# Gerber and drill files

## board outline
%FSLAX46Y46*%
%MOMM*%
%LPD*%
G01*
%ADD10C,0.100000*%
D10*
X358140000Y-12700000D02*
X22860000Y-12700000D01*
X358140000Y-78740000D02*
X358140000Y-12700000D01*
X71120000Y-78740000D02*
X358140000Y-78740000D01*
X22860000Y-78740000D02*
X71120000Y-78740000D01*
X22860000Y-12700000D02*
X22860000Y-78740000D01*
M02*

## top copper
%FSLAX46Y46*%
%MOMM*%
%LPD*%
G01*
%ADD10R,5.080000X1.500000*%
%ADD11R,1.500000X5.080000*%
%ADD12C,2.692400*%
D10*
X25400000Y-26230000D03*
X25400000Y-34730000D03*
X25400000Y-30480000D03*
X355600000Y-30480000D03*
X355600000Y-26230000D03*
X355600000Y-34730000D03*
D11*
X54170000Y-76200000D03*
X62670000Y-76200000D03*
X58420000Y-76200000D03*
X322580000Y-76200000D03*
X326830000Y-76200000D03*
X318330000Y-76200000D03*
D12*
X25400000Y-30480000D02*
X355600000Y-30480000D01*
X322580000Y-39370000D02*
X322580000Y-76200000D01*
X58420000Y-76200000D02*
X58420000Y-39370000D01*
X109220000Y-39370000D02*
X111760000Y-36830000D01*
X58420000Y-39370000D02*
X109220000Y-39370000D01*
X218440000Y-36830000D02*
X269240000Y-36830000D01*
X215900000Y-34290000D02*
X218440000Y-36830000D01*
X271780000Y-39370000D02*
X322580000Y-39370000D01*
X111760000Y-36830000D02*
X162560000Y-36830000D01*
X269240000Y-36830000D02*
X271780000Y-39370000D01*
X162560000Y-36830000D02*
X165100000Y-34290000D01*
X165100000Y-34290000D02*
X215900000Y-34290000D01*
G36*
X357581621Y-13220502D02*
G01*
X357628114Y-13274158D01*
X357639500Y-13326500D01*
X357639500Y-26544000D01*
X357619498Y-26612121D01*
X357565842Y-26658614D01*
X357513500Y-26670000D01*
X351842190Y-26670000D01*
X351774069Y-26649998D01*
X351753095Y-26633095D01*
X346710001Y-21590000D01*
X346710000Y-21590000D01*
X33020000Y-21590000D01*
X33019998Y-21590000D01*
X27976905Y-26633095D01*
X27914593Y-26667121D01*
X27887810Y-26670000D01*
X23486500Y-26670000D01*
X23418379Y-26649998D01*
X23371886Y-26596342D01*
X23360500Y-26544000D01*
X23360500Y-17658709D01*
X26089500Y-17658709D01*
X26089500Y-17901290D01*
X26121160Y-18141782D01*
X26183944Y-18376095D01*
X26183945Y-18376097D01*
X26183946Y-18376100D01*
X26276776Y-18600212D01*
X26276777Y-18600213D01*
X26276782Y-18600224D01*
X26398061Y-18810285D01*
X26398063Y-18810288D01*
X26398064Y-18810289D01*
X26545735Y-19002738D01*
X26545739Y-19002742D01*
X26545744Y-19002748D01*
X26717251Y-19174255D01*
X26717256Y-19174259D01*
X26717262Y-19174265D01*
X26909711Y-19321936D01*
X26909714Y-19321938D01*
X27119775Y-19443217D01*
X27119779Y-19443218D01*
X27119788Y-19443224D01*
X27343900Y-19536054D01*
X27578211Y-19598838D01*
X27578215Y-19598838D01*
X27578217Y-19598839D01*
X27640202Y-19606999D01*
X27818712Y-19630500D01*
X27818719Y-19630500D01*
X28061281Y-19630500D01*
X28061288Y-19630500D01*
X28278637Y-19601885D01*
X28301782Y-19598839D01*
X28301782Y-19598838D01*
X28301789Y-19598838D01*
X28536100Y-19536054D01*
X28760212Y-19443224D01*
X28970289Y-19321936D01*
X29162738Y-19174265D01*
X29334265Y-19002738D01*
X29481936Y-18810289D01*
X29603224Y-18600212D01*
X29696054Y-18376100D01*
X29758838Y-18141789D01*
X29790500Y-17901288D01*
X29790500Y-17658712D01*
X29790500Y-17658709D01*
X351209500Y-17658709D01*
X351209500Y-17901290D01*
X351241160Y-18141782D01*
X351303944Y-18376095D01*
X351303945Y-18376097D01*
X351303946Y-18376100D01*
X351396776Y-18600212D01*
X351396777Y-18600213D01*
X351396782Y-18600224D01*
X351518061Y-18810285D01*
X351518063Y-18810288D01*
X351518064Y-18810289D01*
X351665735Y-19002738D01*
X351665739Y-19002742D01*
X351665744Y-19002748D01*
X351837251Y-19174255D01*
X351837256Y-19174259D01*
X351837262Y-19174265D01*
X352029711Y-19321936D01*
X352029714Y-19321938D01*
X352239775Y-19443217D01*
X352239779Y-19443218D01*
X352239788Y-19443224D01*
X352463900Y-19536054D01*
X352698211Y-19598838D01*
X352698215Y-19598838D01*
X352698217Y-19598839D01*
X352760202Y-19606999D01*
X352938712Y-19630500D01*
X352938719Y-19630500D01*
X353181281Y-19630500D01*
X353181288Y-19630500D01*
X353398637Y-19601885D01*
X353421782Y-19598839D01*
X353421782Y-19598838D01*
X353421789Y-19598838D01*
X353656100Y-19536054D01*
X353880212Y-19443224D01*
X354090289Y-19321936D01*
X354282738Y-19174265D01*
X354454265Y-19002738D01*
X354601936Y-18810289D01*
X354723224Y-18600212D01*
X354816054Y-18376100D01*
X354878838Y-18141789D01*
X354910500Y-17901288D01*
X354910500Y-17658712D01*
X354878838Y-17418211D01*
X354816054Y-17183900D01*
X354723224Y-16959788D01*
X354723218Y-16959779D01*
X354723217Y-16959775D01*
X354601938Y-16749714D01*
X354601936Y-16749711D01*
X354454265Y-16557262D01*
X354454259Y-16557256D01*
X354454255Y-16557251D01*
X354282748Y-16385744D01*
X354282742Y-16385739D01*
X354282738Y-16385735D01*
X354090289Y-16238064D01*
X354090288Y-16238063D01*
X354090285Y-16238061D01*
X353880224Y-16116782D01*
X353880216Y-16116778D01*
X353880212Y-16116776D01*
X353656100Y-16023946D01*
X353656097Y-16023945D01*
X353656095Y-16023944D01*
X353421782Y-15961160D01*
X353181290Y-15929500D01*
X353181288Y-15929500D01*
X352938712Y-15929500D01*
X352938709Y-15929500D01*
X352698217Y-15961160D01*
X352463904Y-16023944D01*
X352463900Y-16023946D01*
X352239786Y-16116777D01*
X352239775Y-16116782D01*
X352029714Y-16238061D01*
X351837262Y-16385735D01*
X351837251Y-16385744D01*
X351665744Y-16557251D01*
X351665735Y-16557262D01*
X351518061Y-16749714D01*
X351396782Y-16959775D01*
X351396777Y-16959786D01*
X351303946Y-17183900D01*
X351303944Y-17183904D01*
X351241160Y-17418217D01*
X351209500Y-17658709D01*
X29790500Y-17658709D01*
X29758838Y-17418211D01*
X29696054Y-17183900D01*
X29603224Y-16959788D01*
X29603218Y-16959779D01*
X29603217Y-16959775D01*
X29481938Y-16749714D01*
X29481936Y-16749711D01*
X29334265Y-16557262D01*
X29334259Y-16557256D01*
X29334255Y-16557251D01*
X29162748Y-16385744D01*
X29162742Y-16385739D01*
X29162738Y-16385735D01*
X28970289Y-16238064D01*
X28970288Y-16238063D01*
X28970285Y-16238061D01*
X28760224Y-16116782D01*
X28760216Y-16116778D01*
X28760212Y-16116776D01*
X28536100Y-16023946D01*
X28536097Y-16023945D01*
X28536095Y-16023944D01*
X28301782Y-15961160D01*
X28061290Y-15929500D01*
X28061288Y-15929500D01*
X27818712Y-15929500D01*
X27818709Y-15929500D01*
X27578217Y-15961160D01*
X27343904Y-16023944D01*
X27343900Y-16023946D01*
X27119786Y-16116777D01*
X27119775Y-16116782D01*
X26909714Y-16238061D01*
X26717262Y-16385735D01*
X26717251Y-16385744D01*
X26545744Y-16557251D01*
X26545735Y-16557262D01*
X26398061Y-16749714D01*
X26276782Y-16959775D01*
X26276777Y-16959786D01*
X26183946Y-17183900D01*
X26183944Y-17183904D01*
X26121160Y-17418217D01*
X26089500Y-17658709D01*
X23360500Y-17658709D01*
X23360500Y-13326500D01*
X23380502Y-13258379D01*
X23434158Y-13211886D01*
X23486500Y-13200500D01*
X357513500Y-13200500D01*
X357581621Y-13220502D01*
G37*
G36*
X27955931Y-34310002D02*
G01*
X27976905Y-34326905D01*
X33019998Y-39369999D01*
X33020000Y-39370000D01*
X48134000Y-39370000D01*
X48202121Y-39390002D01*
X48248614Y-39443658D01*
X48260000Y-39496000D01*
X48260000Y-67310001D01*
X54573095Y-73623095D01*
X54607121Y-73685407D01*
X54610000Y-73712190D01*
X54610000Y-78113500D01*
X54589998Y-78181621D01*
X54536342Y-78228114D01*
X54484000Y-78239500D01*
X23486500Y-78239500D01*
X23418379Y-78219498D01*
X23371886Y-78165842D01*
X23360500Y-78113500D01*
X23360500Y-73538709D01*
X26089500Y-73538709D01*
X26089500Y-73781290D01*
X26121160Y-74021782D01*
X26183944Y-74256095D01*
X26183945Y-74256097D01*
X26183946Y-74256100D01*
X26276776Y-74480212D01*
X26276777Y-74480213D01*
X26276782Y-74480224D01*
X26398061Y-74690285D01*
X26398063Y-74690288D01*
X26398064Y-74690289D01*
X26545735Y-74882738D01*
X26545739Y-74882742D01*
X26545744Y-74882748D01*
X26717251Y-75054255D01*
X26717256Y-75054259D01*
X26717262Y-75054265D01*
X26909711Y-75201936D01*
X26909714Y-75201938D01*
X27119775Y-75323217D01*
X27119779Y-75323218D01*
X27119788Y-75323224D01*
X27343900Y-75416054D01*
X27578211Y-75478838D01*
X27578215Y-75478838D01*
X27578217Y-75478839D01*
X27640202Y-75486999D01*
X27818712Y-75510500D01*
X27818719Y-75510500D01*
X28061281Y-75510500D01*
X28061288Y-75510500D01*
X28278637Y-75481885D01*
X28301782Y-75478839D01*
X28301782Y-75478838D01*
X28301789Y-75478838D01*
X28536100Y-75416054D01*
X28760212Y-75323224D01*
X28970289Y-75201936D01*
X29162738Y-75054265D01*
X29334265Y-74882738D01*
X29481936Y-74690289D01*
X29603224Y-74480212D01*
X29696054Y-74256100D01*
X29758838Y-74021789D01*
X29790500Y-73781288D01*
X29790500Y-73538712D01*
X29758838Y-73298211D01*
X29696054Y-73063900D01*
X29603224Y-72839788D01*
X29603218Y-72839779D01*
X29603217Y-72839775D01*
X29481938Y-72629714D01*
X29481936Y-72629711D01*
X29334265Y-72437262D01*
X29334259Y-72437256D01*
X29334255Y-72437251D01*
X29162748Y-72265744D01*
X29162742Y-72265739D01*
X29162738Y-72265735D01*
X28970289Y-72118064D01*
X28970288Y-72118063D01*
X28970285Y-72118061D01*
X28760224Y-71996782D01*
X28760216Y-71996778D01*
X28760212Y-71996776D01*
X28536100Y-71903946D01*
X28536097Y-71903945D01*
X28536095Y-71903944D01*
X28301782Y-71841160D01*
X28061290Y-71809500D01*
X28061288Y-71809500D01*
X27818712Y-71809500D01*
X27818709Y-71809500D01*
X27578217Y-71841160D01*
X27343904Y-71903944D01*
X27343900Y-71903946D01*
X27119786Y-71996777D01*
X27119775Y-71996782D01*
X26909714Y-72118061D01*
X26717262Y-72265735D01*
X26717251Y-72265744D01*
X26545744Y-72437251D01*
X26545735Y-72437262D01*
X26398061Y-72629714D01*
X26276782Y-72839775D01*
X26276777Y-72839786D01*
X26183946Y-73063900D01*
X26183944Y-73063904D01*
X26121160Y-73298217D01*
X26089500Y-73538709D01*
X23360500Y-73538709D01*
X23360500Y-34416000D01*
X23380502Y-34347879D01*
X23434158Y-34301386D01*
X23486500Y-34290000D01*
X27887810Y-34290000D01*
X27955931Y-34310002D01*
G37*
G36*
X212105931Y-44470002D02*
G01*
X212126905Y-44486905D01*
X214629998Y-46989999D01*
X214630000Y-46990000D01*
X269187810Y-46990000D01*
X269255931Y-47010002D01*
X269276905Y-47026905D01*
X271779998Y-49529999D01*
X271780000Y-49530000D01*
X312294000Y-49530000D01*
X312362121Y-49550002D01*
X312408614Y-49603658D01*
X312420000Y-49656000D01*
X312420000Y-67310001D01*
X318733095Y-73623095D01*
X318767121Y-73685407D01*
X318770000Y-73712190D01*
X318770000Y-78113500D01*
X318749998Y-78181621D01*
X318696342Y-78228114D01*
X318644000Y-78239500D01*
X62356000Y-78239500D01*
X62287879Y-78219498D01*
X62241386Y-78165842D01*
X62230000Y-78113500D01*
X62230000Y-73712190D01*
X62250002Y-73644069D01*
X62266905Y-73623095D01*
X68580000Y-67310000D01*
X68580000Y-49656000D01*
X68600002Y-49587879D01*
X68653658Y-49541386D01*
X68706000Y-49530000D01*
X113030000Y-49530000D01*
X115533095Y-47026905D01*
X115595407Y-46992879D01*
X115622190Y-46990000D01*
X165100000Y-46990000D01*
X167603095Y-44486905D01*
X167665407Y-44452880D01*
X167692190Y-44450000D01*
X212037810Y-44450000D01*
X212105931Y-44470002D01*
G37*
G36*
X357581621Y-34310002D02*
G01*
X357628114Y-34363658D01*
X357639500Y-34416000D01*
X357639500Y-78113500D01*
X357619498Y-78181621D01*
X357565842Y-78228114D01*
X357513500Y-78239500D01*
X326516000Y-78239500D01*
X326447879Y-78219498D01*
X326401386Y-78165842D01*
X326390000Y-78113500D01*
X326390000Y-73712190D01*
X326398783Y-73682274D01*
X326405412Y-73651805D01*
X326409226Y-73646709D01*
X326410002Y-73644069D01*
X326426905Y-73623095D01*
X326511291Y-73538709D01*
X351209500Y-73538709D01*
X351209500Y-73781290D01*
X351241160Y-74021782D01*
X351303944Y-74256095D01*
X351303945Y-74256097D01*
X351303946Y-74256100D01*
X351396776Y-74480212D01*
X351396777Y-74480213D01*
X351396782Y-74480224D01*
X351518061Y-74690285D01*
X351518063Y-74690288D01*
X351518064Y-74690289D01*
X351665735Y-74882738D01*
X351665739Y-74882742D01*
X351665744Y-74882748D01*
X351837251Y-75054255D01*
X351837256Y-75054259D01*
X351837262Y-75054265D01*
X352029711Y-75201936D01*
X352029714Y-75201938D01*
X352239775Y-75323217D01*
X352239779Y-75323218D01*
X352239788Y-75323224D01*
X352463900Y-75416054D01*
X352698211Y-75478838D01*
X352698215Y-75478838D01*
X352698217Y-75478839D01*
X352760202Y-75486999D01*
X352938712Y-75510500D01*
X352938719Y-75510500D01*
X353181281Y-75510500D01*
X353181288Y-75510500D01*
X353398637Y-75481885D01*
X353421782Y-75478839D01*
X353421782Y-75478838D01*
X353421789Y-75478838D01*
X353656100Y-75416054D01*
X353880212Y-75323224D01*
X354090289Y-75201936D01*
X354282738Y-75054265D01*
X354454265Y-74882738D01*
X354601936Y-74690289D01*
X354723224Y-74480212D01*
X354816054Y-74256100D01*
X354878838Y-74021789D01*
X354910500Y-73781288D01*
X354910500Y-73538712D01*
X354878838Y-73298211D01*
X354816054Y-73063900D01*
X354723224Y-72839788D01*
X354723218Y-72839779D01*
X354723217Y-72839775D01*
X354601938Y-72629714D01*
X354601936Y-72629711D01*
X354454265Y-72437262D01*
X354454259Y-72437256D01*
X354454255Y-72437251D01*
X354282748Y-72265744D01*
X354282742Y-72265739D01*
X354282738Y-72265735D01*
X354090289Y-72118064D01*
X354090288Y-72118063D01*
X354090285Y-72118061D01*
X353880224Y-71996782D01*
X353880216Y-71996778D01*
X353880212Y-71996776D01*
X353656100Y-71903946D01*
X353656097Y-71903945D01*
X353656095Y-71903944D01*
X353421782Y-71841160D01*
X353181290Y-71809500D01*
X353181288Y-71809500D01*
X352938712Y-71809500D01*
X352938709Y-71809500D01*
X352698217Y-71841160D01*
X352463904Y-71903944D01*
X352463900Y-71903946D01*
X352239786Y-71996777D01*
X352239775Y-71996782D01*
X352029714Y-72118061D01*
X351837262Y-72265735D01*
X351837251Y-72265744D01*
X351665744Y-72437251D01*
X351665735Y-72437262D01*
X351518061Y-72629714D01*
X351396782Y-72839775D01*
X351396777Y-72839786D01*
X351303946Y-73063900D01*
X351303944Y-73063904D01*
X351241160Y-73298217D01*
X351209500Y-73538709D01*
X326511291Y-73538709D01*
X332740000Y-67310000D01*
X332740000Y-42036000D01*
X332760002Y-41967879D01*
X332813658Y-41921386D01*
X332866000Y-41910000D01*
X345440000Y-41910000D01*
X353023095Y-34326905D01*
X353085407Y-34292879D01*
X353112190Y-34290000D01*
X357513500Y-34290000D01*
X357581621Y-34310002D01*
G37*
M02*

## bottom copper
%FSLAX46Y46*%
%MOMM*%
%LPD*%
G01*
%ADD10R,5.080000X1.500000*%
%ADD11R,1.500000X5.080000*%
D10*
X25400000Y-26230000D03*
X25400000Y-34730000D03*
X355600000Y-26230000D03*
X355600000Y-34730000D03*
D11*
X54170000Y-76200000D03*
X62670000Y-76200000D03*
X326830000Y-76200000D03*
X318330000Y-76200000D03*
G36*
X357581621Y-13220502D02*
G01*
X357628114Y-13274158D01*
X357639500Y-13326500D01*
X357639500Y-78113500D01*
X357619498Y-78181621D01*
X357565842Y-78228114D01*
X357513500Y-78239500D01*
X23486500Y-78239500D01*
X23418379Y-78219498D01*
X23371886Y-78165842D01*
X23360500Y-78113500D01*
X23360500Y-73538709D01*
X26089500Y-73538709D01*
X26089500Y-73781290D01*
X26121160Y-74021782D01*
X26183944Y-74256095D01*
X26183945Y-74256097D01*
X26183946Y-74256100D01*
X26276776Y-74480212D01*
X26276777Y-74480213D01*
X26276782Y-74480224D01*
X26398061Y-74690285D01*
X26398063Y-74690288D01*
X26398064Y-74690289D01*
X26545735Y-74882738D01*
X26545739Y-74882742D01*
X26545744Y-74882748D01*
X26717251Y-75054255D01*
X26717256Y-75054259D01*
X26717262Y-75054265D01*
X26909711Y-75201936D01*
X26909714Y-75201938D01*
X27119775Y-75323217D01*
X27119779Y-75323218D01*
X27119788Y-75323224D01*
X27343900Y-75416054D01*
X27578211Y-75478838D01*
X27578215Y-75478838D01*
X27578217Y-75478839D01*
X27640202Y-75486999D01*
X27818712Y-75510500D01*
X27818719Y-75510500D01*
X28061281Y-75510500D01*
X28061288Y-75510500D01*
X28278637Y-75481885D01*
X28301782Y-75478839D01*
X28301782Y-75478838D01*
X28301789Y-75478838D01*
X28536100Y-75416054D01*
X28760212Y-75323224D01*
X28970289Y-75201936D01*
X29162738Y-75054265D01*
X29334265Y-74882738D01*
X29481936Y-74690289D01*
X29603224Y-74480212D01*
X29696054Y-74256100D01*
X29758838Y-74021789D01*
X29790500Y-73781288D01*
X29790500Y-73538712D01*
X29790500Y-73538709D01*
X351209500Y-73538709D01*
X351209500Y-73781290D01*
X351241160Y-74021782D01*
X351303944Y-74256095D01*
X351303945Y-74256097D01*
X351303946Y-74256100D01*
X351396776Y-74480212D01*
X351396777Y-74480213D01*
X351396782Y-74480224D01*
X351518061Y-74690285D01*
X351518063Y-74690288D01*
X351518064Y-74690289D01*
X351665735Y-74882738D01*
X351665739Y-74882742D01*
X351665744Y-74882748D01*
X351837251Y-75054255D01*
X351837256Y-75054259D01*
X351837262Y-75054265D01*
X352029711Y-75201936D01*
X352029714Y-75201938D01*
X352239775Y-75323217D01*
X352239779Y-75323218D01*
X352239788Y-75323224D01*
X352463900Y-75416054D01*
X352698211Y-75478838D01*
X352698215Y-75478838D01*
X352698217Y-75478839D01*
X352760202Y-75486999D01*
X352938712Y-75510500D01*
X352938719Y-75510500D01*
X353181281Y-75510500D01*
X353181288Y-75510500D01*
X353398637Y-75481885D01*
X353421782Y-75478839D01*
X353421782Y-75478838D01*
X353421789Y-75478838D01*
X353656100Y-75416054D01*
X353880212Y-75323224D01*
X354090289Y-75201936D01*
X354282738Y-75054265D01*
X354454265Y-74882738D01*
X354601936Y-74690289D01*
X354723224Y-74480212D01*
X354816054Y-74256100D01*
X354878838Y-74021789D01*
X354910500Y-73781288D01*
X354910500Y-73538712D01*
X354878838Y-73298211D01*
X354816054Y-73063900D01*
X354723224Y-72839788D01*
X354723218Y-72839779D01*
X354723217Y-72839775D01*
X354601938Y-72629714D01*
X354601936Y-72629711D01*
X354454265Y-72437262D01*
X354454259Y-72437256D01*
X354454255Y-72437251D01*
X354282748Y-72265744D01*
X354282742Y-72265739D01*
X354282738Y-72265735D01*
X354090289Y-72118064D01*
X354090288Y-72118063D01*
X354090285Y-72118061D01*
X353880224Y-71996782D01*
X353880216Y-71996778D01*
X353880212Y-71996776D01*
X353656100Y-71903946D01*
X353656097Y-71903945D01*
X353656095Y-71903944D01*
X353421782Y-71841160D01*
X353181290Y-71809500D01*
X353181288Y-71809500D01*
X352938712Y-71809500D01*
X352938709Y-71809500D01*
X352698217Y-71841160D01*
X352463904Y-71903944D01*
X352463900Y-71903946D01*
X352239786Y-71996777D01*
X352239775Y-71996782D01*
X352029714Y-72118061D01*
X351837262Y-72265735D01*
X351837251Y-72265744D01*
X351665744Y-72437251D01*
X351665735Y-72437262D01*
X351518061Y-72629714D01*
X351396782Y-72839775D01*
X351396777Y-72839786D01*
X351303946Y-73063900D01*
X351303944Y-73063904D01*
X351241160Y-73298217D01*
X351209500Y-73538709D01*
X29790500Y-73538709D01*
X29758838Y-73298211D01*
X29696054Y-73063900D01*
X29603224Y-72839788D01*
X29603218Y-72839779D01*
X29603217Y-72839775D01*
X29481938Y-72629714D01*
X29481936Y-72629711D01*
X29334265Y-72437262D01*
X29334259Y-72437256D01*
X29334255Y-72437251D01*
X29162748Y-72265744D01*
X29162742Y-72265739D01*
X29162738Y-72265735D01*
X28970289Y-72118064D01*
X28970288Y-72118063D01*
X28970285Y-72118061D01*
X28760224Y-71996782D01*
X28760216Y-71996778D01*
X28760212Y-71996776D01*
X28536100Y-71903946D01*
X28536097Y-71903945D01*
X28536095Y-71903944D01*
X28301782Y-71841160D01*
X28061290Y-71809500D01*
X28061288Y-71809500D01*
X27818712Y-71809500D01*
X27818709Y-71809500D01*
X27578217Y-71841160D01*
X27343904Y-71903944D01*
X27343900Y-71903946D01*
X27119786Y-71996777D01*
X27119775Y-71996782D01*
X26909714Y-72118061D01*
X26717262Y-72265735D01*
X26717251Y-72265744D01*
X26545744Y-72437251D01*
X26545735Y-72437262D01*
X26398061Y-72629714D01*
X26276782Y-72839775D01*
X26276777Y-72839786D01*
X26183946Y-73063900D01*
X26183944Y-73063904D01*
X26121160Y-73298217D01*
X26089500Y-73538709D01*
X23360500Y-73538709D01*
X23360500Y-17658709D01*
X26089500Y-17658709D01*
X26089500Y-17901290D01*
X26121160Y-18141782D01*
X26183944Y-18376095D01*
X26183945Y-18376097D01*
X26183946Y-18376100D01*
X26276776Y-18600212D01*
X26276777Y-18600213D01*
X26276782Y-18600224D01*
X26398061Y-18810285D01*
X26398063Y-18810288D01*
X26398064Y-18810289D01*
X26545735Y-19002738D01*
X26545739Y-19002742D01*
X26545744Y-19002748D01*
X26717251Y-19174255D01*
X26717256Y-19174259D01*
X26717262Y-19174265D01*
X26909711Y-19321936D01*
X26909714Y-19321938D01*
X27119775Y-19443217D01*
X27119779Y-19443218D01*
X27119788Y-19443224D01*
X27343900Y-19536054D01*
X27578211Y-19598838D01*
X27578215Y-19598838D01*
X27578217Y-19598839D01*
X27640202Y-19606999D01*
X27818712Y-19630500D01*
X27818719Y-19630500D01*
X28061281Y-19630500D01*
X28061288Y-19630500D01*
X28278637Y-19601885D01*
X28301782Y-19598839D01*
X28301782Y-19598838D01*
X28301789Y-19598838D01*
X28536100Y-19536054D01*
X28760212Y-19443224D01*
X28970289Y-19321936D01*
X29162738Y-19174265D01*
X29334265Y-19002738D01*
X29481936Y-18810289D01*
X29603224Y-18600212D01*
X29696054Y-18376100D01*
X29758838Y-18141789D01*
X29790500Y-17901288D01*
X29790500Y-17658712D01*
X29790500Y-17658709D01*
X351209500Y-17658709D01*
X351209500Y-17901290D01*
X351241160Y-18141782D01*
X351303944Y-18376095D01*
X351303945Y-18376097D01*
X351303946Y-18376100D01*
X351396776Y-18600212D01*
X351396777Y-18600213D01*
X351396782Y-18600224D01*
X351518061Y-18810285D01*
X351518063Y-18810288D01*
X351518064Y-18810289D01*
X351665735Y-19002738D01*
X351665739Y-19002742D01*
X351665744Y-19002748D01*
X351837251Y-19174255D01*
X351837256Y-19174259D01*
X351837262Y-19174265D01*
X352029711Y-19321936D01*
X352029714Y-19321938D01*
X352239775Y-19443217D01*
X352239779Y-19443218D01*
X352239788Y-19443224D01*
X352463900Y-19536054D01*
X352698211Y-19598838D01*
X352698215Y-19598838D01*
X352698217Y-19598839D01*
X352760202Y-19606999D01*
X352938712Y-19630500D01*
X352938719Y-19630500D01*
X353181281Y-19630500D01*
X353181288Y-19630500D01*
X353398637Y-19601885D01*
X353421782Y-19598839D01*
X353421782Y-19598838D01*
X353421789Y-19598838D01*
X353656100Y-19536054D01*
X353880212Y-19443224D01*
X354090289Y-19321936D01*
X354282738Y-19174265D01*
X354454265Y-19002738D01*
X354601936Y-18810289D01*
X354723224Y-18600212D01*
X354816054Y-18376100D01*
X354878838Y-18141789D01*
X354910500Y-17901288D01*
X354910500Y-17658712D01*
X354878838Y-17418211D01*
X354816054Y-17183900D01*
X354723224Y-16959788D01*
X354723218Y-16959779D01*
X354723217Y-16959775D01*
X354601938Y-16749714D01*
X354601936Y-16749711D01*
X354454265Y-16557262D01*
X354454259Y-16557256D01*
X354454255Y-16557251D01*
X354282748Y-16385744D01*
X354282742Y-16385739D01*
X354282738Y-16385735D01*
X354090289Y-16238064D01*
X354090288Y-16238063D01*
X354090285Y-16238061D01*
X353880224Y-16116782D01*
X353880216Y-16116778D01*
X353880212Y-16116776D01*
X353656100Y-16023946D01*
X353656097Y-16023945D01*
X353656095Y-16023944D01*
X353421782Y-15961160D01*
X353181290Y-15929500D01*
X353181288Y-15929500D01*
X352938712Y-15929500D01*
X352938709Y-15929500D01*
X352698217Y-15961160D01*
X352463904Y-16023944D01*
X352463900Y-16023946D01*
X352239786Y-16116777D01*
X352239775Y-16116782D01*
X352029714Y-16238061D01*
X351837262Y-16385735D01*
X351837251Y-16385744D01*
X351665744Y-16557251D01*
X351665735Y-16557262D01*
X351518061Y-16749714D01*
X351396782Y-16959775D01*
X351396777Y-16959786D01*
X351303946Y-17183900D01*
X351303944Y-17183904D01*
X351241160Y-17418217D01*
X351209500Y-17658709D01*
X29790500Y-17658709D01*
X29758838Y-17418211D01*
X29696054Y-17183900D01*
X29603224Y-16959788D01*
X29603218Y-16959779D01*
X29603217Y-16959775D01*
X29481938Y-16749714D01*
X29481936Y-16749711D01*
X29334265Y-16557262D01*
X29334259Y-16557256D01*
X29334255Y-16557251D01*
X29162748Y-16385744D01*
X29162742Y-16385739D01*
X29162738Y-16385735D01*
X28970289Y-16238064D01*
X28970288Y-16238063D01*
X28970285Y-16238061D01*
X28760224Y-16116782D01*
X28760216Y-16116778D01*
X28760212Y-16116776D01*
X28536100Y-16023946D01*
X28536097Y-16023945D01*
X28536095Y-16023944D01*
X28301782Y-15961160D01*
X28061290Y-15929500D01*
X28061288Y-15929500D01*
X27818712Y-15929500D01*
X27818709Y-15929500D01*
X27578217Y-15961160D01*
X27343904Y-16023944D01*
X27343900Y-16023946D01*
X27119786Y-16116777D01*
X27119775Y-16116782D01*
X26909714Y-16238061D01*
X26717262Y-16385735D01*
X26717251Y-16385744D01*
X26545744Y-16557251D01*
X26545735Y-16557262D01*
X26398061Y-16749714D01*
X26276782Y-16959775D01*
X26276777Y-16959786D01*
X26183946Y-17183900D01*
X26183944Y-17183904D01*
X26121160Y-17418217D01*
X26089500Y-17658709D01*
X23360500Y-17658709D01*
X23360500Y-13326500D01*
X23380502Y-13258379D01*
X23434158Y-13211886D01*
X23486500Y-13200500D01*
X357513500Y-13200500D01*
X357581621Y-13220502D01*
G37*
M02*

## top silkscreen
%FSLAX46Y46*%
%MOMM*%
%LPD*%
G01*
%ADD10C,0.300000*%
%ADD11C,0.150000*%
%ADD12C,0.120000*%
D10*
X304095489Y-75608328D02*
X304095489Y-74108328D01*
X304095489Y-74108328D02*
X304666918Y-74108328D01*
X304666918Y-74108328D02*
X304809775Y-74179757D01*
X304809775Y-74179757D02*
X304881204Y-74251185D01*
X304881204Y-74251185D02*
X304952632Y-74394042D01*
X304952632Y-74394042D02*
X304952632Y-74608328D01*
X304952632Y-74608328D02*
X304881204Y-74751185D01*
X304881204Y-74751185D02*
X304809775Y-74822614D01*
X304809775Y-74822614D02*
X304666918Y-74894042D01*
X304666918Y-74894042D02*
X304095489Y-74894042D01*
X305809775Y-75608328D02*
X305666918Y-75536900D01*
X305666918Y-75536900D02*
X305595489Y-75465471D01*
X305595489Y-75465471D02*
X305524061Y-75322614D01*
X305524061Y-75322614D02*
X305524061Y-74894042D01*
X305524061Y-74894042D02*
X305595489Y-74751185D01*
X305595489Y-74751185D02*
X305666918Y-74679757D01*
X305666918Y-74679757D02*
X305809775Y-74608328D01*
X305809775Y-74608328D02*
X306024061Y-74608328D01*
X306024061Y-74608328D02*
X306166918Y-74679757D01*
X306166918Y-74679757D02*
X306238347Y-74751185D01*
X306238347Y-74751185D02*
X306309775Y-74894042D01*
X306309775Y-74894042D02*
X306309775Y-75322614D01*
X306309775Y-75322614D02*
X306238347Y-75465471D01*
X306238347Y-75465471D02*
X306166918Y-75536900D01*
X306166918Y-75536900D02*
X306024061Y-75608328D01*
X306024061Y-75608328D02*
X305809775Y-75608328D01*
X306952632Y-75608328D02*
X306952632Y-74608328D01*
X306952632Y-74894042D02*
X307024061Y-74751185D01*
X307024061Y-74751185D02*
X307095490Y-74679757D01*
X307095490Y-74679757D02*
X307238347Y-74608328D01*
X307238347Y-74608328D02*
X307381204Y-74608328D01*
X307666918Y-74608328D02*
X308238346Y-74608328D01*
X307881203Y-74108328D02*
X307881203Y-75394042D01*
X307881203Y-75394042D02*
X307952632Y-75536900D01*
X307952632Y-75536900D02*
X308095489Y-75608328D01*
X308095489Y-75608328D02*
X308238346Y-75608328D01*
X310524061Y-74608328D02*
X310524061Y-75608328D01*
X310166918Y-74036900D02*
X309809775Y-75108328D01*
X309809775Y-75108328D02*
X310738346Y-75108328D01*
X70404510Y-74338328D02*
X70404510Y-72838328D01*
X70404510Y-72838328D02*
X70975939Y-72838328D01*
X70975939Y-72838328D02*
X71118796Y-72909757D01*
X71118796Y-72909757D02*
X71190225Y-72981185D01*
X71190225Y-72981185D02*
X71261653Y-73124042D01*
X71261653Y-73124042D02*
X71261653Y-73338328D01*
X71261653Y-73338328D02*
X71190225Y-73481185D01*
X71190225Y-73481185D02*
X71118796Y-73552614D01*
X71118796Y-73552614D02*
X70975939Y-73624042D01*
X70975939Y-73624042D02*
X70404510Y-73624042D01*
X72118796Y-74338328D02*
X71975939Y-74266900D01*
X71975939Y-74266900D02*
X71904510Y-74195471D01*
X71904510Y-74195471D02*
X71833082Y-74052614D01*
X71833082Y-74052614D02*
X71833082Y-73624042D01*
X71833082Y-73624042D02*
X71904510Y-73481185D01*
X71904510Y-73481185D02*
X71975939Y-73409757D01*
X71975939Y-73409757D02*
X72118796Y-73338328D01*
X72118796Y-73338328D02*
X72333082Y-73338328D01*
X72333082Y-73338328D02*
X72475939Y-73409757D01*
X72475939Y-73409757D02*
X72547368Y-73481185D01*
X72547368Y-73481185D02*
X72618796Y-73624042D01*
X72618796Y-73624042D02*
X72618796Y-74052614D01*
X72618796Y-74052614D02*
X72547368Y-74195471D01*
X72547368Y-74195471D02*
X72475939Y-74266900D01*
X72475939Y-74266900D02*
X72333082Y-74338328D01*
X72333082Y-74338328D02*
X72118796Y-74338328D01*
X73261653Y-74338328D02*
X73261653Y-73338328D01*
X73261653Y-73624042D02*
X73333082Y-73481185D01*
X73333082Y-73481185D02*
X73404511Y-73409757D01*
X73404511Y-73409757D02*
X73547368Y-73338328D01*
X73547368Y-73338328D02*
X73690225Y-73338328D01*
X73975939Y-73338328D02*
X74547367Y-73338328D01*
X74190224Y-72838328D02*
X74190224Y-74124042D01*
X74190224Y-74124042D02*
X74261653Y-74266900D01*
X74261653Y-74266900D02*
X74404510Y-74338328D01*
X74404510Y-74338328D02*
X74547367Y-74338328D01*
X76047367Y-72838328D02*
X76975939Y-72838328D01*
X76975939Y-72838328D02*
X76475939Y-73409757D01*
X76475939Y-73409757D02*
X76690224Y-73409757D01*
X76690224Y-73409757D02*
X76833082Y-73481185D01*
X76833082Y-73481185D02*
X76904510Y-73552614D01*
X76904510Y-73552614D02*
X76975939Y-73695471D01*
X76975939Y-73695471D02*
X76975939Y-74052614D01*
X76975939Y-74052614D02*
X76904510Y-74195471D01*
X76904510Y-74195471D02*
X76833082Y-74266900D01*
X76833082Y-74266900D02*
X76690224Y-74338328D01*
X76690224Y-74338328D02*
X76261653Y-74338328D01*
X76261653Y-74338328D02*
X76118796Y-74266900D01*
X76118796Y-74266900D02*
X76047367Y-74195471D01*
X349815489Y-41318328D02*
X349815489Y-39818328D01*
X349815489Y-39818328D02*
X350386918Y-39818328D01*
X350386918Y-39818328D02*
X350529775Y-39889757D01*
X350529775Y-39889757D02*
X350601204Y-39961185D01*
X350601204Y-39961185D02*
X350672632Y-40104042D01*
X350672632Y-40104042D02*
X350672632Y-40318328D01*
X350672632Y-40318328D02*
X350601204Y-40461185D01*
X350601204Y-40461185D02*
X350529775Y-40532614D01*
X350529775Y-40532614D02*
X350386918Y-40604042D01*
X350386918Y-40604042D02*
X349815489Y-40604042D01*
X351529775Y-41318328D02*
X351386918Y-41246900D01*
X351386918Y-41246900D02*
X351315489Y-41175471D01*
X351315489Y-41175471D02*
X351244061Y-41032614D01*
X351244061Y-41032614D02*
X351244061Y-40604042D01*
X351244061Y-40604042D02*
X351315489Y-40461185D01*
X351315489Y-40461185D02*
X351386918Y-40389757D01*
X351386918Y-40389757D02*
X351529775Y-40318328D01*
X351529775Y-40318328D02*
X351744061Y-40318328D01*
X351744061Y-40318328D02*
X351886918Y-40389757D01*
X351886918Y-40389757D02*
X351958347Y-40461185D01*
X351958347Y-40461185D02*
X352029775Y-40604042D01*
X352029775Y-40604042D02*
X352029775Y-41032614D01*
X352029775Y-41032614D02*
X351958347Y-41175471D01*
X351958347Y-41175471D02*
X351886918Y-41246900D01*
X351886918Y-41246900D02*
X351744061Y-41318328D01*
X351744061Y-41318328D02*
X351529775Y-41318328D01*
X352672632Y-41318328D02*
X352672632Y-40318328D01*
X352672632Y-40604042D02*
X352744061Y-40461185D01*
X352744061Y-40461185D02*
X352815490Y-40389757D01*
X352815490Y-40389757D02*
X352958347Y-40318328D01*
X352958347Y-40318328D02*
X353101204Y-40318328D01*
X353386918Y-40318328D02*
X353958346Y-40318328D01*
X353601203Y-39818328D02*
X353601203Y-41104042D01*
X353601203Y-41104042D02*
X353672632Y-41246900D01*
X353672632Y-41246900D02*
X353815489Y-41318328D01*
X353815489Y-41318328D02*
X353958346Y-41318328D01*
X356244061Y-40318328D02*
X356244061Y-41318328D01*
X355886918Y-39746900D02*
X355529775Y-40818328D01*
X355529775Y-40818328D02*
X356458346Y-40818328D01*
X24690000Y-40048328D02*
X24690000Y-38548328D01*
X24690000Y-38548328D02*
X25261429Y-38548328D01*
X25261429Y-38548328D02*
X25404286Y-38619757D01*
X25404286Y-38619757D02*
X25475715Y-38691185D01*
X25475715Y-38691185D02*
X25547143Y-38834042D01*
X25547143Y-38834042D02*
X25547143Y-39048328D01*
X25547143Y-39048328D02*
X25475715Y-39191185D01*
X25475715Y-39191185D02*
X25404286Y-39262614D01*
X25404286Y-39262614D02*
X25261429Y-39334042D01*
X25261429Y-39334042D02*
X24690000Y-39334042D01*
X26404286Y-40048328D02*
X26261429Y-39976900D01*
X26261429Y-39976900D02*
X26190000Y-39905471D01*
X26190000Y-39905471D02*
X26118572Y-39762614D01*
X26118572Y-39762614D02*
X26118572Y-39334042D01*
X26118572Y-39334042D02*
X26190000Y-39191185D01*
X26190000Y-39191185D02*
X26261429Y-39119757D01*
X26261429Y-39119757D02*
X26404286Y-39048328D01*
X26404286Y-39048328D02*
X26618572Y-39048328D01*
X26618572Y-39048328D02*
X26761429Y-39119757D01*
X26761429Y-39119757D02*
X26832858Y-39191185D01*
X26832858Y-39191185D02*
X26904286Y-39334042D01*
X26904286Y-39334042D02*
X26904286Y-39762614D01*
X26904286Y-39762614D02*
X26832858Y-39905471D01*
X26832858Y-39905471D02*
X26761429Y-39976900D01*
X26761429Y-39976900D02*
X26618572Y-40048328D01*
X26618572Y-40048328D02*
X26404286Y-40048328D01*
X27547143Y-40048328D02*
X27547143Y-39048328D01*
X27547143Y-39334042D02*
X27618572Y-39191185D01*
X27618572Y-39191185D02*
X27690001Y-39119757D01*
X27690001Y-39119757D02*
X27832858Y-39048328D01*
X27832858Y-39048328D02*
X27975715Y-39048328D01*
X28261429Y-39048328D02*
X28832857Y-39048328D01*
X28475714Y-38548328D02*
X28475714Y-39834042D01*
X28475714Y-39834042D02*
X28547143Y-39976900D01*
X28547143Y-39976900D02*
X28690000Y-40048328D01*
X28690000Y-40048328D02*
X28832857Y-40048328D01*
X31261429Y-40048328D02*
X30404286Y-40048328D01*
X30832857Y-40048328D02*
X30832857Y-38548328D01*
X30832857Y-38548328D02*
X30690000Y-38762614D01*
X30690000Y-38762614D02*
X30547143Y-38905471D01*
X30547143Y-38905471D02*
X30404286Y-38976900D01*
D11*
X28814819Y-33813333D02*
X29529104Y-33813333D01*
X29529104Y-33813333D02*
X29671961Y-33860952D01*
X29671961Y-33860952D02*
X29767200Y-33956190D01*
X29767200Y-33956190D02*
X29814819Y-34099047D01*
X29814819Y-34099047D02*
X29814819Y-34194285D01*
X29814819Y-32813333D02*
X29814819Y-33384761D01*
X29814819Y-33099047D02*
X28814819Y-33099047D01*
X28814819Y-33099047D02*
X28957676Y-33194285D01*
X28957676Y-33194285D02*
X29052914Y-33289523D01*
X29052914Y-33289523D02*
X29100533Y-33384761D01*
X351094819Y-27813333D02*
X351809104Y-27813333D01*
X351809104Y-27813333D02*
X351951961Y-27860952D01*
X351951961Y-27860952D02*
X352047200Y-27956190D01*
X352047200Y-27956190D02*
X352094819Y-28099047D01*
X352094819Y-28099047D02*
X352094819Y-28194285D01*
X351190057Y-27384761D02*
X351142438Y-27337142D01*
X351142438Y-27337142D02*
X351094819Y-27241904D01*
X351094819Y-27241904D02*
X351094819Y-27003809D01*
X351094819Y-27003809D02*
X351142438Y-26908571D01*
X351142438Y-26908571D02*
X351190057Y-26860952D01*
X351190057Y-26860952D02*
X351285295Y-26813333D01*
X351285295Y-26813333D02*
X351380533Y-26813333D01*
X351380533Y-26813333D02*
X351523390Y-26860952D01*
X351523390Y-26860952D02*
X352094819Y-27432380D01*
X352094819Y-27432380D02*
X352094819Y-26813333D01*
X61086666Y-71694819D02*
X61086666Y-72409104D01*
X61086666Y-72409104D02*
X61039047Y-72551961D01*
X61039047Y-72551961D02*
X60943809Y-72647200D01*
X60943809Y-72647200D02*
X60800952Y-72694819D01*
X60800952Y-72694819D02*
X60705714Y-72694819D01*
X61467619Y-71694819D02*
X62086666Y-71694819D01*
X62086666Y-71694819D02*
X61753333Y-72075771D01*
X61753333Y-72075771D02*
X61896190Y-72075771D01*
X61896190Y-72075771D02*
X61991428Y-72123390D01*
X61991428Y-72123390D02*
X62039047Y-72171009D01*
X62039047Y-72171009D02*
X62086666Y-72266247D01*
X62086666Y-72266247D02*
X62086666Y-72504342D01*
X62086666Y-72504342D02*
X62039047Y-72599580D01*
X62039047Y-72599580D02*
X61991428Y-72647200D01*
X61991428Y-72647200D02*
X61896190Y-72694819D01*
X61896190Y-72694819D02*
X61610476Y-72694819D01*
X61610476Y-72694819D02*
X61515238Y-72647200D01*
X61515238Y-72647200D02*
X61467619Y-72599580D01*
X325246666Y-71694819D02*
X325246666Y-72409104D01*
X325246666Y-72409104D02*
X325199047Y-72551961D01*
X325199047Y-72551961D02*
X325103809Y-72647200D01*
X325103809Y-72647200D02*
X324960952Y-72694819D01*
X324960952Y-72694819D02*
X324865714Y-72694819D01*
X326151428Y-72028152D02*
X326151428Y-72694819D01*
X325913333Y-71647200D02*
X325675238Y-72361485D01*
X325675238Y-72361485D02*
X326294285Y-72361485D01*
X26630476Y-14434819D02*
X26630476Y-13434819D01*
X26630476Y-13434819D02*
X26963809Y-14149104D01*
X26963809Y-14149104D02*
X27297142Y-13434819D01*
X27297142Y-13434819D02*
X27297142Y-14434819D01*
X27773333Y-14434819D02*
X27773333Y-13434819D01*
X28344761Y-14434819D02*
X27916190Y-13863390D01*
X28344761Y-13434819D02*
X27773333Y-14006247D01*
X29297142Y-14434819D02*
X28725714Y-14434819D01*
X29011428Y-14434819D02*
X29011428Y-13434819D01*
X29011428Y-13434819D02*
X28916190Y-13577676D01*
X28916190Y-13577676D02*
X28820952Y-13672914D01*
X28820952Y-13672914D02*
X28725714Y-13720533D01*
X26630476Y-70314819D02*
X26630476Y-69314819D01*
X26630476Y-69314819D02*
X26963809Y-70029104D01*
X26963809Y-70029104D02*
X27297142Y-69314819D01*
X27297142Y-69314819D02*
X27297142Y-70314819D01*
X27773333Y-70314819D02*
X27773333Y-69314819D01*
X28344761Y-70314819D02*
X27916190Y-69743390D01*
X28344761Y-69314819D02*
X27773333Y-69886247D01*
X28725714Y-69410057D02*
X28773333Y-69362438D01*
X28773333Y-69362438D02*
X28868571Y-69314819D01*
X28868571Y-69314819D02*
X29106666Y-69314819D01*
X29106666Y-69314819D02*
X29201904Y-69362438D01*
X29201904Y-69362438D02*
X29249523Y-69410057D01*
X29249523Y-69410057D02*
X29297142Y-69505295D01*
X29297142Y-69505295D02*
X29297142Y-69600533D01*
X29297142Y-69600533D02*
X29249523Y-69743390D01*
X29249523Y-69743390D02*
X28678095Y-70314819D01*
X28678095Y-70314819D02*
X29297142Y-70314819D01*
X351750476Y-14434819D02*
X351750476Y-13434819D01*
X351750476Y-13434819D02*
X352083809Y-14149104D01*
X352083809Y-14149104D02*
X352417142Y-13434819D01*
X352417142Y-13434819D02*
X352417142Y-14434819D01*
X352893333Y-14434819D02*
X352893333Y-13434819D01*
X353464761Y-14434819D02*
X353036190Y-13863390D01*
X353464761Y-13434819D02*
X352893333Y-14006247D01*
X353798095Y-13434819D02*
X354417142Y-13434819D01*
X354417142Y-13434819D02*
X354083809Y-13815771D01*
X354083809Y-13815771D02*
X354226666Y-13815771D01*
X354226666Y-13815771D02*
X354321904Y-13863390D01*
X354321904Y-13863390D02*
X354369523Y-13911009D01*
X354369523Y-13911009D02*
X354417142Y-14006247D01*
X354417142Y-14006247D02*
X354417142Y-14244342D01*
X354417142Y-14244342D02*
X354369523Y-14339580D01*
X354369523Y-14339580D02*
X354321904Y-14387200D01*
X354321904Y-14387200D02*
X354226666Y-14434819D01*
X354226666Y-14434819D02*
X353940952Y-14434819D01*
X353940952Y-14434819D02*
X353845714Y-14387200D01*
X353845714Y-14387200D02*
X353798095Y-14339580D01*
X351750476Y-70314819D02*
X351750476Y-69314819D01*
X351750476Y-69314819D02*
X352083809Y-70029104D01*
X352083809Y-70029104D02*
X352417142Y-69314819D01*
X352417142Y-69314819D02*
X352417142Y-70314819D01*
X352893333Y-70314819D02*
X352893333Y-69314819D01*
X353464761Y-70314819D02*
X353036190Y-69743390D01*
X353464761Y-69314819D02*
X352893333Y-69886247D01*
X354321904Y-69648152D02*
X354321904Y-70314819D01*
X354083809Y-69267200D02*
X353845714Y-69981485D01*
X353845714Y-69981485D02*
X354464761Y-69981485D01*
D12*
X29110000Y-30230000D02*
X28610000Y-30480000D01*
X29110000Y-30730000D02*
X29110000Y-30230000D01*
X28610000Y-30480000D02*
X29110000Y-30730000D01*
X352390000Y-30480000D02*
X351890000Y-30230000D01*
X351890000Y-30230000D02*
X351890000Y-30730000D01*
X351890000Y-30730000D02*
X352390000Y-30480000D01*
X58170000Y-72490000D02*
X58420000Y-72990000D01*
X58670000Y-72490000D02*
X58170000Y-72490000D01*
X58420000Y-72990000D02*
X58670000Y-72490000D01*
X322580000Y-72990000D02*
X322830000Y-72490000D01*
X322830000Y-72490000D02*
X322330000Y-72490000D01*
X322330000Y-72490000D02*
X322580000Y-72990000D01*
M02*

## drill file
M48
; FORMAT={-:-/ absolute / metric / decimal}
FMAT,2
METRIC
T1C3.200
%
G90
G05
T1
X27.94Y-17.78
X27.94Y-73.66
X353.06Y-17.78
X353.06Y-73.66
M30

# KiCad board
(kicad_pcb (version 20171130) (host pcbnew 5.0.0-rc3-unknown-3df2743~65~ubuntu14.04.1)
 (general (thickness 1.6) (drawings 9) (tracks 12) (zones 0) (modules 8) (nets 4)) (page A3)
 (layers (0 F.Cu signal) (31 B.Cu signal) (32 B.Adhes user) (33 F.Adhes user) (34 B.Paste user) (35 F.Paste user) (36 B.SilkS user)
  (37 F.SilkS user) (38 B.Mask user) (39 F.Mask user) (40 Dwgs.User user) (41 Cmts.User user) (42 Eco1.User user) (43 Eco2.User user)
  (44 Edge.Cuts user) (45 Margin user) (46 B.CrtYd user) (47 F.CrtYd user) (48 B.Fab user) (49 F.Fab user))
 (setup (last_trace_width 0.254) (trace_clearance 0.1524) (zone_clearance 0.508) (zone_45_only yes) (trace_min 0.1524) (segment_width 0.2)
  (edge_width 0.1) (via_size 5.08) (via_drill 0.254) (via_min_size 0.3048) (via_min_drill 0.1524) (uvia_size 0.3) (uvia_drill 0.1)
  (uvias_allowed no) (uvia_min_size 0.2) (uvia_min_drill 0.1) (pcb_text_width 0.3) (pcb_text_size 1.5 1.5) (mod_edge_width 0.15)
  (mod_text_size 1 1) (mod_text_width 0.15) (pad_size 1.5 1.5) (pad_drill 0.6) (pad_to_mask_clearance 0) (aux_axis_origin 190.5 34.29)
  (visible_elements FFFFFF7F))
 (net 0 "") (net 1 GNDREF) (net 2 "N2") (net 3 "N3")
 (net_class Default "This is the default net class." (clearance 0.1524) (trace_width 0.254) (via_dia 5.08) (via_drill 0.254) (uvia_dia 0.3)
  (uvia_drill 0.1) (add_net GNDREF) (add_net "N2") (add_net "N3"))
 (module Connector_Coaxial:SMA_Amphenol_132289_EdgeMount (layer F.Cu) (at 25.4 30.48 180)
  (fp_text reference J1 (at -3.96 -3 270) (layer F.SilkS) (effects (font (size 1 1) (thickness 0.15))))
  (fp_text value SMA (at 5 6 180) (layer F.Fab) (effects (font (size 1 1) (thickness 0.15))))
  (fp_line (start -3.71 0.25) (end -3.21 0) (layer F.SilkS) (width 0.12))
  (fp_line (start -3.71 -0.25) (end -3.71 0.25) (layer F.SilkS) (width 0.12))
  (fp_line (start -3.21 0) (end -3.71 -0.25) (layer F.SilkS) (width 0.12))
  (pad 2 smd rect (at 0 4.25 270) (size 1.5 5.08) (layers B.Cu B.Paste B.Mask) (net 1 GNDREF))
  (pad 2 smd rect (at 0 -4.25 270) (size 1.5 5.08) (layers B.Cu B.Paste B.Mask) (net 1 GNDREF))
  (pad 2 smd rect (at 0 4.25 270) (size 1.5 5.08) (layers F.Cu F.Paste F.Mask) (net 1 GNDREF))
  (pad 2 smd rect (at 0 -4.25 270) (size 1.5 5.08) (layers F.Cu F.Paste F.Mask) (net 1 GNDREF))
  (pad 1 smd rect (at 0 0 270) (size 1.5 5.08) (layers F.Cu F.Paste F.Mask) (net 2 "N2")))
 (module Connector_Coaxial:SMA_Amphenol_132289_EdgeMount (layer F.Cu) (at 355.6 30.48)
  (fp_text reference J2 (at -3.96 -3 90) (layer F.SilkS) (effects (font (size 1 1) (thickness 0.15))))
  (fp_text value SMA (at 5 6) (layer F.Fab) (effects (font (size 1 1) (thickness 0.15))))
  (fp_line (start -3.21 0) (end -3.71 -0.25) (layer F.SilkS) (width 0.12))
  (fp_line (start -3.71 -0.25) (end -3.71 0.25) (layer F.SilkS) (width 0.12))
  (fp_line (start -3.71 0.25) (end -3.21 0) (layer F.SilkS) (width 0.12))
  (pad 1 smd rect (at 0 0 90) (size 1.5 5.08) (layers F.Cu F.Paste F.Mask) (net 2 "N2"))
  (pad 2 smd rect (at 0 -4.25 90) (size 1.5 5.08) (layers F.Cu F.Paste F.Mask) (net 1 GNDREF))
  (pad 2 smd rect (at 0 4.25 90) (size 1.5 5.08) (layers F.Cu F.Paste F.Mask) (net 1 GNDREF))
  (pad 2 smd rect (at 0 -4.25 90) (size 1.5 5.08) (layers B.Cu B.Paste B.Mask) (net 1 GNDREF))
  (pad 2 smd rect (at 0 4.25 90) (size 1.5 5.08) (layers B.Cu B.Paste B.Mask) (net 1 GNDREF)))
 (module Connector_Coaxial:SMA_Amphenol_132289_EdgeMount (layer F.Cu) (at 58.42 76.2 270)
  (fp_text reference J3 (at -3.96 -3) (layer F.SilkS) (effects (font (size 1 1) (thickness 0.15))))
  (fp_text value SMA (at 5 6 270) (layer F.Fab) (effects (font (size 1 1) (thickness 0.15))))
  (fp_line (start -3.71 0.25) (end -3.21 0) (layer F.SilkS) (width 0.12))
  (fp_line (start -3.71 -0.25) (end -3.71 0.25) (layer F.SilkS) (width 0.12))
  (fp_line (start -3.21 0) (end -3.71 -0.25) (layer F.SilkS) (width 0.12))
  (pad 2 smd rect (at 0 4.25) (size 1.5 5.08) (layers B.Cu B.Paste B.Mask) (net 1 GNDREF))
  (pad 2 smd rect (at 0 -4.25) (size 1.5 5.08) (layers B.Cu B.Paste B.Mask) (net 1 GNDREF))
  (pad 2 smd rect (at 0 4.25) (size 1.5 5.08) (layers F.Cu F.Paste F.Mask) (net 1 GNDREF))
  (pad 2 smd rect (at 0 -4.25) (size 1.5 5.08) (layers F.Cu F.Paste F.Mask) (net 1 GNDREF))
  (pad 1 smd rect (at 0 0) (size 1.5 5.08) (layers F.Cu F.Paste F.Mask) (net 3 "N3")))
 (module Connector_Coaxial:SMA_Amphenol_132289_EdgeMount (layer F.Cu) (at 322.58 76.2 270)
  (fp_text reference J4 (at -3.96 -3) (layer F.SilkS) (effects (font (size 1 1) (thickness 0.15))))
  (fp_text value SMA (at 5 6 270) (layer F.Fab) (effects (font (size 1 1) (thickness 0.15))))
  (fp_line (start -3.21 0) (end -3.71 -0.25) (layer F.SilkS) (width 0.12))
  (fp_line (start -3.71 -0.25) (end -3.71 0.25) (layer F.SilkS) (width 0.12))
  (fp_line (start -3.71 0.25) (end -3.21 0) (layer F.SilkS) (width 0.12))
  (pad 1 smd rect (at 0 0) (size 1.5 5.08) (layers F.Cu F.Paste F.Mask) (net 3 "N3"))
  (pad 2 smd rect (at 0 -4.25) (size 1.5 5.08) (layers F.Cu F.Paste F.Mask) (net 1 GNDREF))
  (pad 2 smd rect (at 0 4.25) (size 1.5 5.08) (layers F.Cu F.Paste F.Mask) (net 1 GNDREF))
  (pad 2 smd rect (at 0 -4.25) (size 1.5 5.08) (layers B.Cu B.Paste B.Mask) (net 1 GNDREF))
  (pad 2 smd rect (at 0 4.25) (size 1.5 5.08) (layers B.Cu B.Paste B.Mask) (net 1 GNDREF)))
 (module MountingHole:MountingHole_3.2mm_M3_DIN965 (layer F.Cu) (at 27.94 17.78)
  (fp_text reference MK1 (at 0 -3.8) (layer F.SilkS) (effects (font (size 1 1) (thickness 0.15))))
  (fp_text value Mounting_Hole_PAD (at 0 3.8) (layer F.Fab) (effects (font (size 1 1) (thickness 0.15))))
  (pad 1 np_thru_hole circle (at 0 0) (size 3.2 3.2) (drill 3.2) (layers *.Cu *.Mask) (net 1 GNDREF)))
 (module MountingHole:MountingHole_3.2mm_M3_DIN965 (layer F.Cu) (at 27.94 73.66)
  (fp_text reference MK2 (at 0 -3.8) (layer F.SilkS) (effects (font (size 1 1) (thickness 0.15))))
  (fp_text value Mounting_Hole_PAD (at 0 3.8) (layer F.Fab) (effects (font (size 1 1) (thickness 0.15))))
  (pad 1 np_thru_hole circle (at 0 0) (size 3.2 3.2) (drill 3.2) (layers *.Cu *.Mask) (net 1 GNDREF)))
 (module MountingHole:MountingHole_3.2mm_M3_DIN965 (layer F.Cu) (at 353.06 17.78)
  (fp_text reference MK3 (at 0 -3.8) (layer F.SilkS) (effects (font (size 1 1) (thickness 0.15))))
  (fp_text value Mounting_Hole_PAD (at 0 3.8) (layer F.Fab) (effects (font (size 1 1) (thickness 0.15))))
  (pad 1 np_thru_hole circle (at 0 0) (size 3.2 3.2) (drill 3.2) (layers *.Cu *.Mask) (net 1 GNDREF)))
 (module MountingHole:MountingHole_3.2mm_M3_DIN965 (layer F.Cu) (at 353.06 73.66)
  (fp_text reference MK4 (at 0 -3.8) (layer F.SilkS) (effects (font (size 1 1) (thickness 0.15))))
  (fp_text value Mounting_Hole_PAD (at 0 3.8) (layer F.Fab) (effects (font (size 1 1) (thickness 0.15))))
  (pad 1 np_thru_hole circle (at 0 0) (size 3.2 3.2) (drill 3.2) (layers *.Cu *.Mask) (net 1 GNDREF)))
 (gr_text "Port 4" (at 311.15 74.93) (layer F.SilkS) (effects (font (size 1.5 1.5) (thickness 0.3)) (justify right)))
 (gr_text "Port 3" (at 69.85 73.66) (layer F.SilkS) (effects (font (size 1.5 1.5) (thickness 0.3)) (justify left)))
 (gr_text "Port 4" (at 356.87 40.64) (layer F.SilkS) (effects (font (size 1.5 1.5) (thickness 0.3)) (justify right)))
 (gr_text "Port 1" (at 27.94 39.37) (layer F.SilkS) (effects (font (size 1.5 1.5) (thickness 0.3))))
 (gr_line (start 358.14 12.7) (end 22.86 12.7) (layer Edge.Cuts) (width 0.1))
 (gr_line (start 358.14 78.74) (end 358.14 12.7) (layer Edge.Cuts) (width 0.1))
 (gr_line (start 71.12 78.74) (end 358.14 78.74) (layer Edge.Cuts) (width 0.1))
 (gr_line (start 22.86 78.74) (end 71.12 78.74) (layer Edge.Cuts) (width 0.1))
 (gr_line (start 22.86 12.7) (end 22.86 78.74) (layer Edge.Cuts) (width 0.1))
 (segment (start 25.4 30.48) (end 355.6 30.48) (width 2.6924) (layer F.Cu) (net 2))
 (segment (start 322.58 39.37) (end 322.58 76.2) (width 2.6924) (layer F.Cu) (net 3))
 (segment (start 58.42 76.2) (end 58.42 39.37) (width 2.6924) (layer F.Cu) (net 3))
 (segment (start 109.22 39.37) (end 111.76 36.83) (width 2.6924) (layer F.Cu) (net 3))
 (segment (start 58.42 39.37) (end 109.22 39.37) (width 2.6924) (layer F.Cu) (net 3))
 (segment (start 218.44 36.83) (end 269.24 36.83) (width 2.6924) (layer F.Cu) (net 3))
 (segment (start 215.9 34.29) (end 218.44 36.83) (width 2.6924) (layer F.Cu) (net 3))
 (segment (start 271.78 39.37) (end 322.58 39.37) (width 2.6924) (layer F.Cu) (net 3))
 (segment (start 111.76 36.83) (end 162.56 36.83) (width 2.6924) (layer F.Cu) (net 3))
 (segment (start 269.24 36.83) (end 271.78 39.37) (width 2.6924) (layer F.Cu) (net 3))
 (segment (start 162.56 36.83) (end 165.1 34.29) (width 2.6924) (layer F.Cu) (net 3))
 (segment (start 165.1 34.29) (end 215.9 34.29) (width 2.6924) (layer F.Cu) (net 3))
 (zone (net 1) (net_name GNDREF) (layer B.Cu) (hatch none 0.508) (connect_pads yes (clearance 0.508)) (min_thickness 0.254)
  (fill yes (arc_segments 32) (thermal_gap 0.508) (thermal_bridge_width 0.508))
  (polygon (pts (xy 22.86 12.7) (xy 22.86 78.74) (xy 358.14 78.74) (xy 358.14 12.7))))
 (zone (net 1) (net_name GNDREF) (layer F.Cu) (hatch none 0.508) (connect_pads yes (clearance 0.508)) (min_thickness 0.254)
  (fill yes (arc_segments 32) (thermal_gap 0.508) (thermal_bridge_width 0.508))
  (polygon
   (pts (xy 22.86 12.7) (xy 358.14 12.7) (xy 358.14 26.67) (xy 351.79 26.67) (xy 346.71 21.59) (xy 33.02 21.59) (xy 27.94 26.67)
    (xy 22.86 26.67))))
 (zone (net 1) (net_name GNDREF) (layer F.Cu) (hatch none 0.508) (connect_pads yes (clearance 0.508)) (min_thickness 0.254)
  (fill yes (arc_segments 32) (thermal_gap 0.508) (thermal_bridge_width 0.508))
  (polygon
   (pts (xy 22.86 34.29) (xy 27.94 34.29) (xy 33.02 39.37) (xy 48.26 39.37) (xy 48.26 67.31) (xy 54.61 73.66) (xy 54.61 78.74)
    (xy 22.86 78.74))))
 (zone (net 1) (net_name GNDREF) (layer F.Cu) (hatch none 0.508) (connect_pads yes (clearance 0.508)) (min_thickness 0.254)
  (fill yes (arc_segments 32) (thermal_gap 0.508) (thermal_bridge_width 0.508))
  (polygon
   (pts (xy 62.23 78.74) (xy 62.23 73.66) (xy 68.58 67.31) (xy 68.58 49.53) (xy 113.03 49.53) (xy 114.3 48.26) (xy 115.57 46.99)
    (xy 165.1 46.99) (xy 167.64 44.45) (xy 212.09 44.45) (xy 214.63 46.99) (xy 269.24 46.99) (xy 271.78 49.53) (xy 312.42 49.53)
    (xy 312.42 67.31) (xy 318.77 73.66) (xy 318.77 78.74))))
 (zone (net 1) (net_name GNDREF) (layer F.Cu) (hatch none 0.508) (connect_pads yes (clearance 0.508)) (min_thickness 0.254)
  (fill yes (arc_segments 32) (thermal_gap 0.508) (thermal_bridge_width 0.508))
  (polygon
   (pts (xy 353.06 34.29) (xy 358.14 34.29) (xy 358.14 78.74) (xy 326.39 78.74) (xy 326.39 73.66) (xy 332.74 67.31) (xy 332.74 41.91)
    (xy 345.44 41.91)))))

